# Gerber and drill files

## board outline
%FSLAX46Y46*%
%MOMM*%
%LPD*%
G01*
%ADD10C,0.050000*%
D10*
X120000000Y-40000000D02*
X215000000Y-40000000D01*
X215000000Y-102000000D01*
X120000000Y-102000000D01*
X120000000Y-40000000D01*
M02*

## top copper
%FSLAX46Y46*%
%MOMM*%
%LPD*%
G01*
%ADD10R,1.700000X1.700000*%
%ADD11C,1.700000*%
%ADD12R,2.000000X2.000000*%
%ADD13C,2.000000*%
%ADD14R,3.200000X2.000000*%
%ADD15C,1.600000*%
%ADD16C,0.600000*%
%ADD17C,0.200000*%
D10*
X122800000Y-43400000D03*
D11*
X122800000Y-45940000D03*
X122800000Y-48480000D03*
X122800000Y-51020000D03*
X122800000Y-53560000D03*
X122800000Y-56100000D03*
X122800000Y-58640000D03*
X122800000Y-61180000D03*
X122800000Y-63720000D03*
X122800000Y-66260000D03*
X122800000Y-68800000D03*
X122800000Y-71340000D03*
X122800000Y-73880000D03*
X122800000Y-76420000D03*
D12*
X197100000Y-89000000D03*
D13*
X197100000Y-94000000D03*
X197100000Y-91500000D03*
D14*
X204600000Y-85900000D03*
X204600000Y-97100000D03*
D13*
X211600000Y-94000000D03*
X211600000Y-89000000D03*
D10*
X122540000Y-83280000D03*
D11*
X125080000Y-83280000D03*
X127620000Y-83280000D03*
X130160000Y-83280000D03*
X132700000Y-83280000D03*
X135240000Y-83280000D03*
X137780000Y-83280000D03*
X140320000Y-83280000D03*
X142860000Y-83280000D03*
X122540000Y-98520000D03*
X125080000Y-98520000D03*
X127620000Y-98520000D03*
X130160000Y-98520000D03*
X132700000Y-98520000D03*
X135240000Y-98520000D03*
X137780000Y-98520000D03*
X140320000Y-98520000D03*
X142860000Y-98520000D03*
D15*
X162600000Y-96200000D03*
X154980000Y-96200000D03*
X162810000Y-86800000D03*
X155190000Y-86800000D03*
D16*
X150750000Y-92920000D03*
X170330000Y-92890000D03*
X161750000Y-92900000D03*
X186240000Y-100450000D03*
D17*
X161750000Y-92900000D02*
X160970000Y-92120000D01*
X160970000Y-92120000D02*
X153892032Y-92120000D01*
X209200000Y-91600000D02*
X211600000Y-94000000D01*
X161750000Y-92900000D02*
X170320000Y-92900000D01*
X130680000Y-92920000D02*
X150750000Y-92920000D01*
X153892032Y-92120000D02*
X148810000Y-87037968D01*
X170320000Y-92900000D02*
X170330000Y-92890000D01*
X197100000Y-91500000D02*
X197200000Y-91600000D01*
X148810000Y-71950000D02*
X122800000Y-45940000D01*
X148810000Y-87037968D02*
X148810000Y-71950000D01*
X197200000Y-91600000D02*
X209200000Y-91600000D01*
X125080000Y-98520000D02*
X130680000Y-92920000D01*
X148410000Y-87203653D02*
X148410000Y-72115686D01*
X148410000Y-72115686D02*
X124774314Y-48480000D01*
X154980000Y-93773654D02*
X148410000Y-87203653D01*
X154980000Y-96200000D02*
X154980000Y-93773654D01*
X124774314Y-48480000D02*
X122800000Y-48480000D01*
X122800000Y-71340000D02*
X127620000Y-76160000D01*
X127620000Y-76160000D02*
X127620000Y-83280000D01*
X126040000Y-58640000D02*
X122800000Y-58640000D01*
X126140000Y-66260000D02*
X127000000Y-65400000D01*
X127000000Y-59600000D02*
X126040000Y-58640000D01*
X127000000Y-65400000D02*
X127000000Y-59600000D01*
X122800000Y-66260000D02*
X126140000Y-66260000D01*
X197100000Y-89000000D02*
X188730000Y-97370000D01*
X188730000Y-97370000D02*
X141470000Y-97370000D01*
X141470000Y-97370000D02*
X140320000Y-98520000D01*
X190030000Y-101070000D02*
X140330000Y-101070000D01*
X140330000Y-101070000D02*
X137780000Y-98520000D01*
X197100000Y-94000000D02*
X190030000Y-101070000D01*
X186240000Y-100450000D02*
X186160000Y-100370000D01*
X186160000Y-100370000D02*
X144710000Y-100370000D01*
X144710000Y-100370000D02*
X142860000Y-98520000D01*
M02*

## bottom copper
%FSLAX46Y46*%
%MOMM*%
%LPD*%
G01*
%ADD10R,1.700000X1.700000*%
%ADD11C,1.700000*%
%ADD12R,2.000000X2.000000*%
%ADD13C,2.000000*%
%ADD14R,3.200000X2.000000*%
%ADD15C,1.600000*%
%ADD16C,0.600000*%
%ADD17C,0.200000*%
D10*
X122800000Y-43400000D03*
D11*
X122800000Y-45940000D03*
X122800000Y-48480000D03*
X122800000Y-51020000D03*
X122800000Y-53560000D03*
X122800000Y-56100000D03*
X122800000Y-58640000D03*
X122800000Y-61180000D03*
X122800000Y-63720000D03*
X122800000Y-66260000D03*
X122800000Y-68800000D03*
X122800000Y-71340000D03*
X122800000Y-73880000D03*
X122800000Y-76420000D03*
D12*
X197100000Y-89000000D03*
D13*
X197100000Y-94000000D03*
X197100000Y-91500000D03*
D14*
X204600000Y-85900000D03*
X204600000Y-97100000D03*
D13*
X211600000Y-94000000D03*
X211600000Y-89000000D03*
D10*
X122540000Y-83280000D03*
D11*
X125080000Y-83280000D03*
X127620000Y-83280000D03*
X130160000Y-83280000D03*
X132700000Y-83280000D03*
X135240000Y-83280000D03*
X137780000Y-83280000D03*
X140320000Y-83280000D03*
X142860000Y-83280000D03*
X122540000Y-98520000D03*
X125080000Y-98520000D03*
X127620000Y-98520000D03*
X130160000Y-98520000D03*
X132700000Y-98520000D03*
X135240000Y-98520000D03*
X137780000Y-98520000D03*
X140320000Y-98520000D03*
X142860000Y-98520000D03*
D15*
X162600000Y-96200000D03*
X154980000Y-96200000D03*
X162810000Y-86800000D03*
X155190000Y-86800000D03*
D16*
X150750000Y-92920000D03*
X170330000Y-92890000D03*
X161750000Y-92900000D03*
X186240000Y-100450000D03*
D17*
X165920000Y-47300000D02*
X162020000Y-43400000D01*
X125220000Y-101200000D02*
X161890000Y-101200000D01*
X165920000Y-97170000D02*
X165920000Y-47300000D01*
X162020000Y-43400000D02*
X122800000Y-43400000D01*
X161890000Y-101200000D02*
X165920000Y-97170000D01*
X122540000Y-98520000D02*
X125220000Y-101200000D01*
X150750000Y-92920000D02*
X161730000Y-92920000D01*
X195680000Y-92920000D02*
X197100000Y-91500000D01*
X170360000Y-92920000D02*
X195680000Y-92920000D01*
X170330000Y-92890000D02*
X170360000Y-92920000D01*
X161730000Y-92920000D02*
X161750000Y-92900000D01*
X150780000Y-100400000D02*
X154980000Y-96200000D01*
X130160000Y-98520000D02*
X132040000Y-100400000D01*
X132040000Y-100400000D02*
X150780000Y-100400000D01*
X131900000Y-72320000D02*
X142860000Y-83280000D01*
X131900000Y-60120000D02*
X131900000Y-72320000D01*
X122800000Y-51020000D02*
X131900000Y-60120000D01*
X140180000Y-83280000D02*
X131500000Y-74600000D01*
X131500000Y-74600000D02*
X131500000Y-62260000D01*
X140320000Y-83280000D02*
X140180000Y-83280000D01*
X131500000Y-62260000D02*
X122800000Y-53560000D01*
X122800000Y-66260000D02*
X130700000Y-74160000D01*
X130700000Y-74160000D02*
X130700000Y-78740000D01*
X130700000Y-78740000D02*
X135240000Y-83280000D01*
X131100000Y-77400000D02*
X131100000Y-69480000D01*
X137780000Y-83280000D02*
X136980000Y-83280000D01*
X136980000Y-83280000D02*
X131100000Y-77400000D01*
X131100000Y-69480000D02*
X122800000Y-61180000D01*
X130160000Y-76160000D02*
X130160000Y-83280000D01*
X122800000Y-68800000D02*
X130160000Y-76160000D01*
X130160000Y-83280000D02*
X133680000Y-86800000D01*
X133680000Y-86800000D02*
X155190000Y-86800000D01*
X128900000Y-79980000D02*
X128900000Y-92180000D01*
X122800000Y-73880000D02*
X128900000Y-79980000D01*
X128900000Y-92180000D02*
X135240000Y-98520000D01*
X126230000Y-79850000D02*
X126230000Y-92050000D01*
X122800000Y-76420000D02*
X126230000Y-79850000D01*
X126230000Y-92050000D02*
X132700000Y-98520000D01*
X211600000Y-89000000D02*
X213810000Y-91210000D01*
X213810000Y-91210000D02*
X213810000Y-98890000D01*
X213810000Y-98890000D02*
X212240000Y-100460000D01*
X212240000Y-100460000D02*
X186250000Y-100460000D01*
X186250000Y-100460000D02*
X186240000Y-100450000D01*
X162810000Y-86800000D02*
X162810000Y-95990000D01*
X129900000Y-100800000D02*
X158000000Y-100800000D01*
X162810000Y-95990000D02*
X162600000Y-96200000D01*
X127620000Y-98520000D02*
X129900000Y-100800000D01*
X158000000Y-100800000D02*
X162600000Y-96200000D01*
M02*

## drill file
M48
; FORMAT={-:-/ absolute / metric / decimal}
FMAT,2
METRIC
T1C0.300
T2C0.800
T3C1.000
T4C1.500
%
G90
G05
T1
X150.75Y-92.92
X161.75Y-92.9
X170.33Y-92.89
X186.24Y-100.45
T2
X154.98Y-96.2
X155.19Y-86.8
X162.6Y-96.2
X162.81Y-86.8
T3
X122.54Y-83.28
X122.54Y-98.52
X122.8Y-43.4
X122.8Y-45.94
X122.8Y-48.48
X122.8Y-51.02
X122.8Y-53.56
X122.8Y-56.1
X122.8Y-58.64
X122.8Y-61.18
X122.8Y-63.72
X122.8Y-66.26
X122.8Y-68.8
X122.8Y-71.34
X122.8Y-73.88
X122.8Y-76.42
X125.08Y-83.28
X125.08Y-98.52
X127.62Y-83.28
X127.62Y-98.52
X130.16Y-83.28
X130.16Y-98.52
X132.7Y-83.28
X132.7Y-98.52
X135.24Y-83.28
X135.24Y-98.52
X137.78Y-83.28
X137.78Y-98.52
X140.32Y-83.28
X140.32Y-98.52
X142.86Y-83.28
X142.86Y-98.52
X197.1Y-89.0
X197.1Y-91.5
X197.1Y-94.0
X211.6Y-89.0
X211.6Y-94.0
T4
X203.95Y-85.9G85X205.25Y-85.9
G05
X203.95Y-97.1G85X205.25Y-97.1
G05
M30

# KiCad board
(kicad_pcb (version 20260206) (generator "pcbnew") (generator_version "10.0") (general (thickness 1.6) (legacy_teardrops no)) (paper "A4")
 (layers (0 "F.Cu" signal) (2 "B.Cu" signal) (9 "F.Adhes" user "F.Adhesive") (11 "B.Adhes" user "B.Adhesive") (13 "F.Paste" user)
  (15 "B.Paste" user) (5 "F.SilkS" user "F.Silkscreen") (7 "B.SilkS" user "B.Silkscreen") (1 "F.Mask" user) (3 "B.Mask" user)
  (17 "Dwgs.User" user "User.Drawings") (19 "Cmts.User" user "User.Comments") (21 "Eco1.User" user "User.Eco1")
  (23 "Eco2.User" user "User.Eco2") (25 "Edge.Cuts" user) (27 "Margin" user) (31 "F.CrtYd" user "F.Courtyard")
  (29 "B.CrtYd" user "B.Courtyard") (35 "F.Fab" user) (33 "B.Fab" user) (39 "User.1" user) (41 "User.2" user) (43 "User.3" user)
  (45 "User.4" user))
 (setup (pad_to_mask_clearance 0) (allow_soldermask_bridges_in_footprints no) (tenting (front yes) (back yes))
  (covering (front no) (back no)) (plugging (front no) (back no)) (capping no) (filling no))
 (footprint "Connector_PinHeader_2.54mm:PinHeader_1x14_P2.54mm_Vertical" (layer "F.Cu") (at 122.8 43.4)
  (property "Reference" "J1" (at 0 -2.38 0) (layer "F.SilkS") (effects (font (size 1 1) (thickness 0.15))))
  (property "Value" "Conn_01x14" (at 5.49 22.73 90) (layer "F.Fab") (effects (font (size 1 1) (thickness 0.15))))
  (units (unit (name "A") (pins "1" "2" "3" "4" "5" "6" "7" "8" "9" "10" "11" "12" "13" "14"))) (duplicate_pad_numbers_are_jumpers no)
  (pad "1" thru_hole rect (at 0 0) (size 1.7 1.7) (drill 1) (layers "*.Cu" "*.Mask") (remove_unused_layers no) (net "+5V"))
  (pad "2" thru_hole circle (at 0 2.54) (size 1.7 1.7) (drill 1) (layers "*.Cu" "*.Mask") (remove_unused_layers no) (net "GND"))
  (pad "3" thru_hole circle (at 0 5.08) (size 1.7 1.7) (drill 1) (layers "*.Cu" "*.Mask") (remove_unused_layers no) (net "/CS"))
  (pad "4" thru_hole circle (at 0 7.62) (size 1.7 1.7) (drill 1) (layers "*.Cu" "*.Mask") (remove_unused_layers no) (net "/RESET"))
  (pad "5" thru_hole circle (at 0 10.16) (size 1.7 1.7) (drill 1) (layers "*.Cu" "*.Mask") (remove_unused_layers no) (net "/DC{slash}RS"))
  (pad "6" thru_hole circle (at 0 12.7) (size 1.7 1.7) (drill 1) (layers "*.Cu" "*.Mask") (remove_unused_layers no) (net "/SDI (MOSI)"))
  (pad "7" thru_hole circle (at 0 15.24) (size 1.7 1.7) (drill 1) (layers "*.Cu" "*.Mask") (remove_unused_layers no) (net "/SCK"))
  (pad "8" thru_hole circle (at 0 17.78) (size 1.7 1.7) (drill 1) (layers "*.Cu" "*.Mask") (remove_unused_layers no) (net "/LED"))
  (pad "9" thru_hole circle (at 0 20.32) (size 1.7 1.7) (drill 1) (layers "*.Cu" "*.Mask") (remove_unused_layers no)
   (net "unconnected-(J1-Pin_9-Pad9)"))
  (pad "10" thru_hole circle (at 0 22.86) (size 1.7 1.7) (drill 1) (layers "*.Cu" "*.Mask") (remove_unused_layers no) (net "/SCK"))
  (pad "11" thru_hole circle (at 0 25.4) (size 1.7 1.7) (drill 1) (layers "*.Cu" "*.Mask") (remove_unused_layers no) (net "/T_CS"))
  (pad "12" thru_hole circle (at 0 27.94) (size 1.7 1.7) (drill 1) (layers "*.Cu" "*.Mask") (remove_unused_layers no) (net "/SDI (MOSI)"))
  (pad "13" thru_hole circle (at 0 30.48) (size 1.7 1.7) (drill 1) (layers "*.Cu" "*.Mask") (remove_unused_layers no) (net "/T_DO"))
  (pad "14" thru_hole circle (at 0 33.02) (size 1.7 1.7) (drill 1) (layers "*.Cu" "*.Mask") (remove_unused_layers no) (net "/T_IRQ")))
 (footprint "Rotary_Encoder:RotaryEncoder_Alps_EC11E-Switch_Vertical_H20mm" (layer "F.Cu") (at 197.1 89)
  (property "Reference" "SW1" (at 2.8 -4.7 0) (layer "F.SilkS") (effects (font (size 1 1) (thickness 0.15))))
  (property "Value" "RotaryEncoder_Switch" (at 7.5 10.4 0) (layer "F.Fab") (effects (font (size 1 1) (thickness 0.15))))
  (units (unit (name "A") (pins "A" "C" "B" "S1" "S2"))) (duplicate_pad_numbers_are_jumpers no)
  (pad "A" thru_hole rect (at 0 0) (size 2 2) (drill 1) (layers "*.Cu" "*.Mask") (remove_unused_layers no) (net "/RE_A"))
  (pad "B" thru_hole circle (at 0 5) (size 2 2) (drill 1) (layers "*.Cu" "*.Mask") (remove_unused_layers no) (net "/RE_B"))
  (pad "C" thru_hole circle (at 0 2.5) (size 2 2) (drill 1) (layers "*.Cu" "*.Mask") (remove_unused_layers no) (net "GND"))
  (pad "MP" thru_hole rect (at 7.5 -3.1) (size 3.2 2) (drill oval 2.8 1.5) (layers "*.Cu" "*.Mask") (remove_unused_layers no))
  (pad "MP" thru_hole rect (at 7.5 8.1) (size 3.2 2) (drill oval 2.8 1.5) (layers "*.Cu" "*.Mask") (remove_unused_layers no))
  (pad "S1" thru_hole circle (at 14.5 5) (size 2 2) (drill 1) (layers "*.Cu" "*.Mask") (remove_unused_layers no) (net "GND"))
  (pad "S2" thru_hole circle (at 14.5 0) (size 2 2) (drill 1) (layers "*.Cu" "*.Mask") (remove_unused_layers no) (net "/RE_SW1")))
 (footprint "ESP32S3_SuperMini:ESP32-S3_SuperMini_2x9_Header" (layer "B.Cu") (at 132.7 90.9 -90)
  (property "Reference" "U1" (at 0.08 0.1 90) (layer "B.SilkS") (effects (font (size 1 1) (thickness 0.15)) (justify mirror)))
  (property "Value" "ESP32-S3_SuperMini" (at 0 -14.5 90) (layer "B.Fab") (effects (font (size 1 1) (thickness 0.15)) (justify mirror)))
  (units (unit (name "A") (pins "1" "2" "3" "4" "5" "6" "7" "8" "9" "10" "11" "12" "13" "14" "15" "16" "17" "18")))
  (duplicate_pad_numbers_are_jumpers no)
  (pad "1" thru_hole rect (at -7.62 10.16 270) (size 1.7 1.7) (drill 1) (layers "*.Cu" "*.Mask") (remove_unused_layers no)
   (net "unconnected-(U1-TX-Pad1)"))
  (pad "2" thru_hole circle (at -7.62 7.62 270) (size 1.7 1.7) (drill 1) (layers "*.Cu" "*.Mask") (remove_unused_layers no)
   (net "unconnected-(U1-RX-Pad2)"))
  (pad "3" thru_hole circle (at -7.62 5.08 270) (size 1.7 1.7) (drill 1) (layers "*.Cu" "*.Mask") (remove_unused_layers no)
   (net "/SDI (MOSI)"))
  (pad "4" thru_hole circle (at -7.62 2.54 270) (size 1.7 1.7) (drill 1) (layers "*.Cu" "*.Mask") (remove_unused_layers no) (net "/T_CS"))
  (pad "5" thru_hole circle (at -7.62 0 270) (size 1.7 1.7) (drill 1) (layers "*.Cu" "*.Mask") (remove_unused_layers no)
   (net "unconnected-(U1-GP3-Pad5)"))
  (pad "6" thru_hole circle (at -7.62 -2.54 270) (size 1.7 1.7) (drill 1) (layers "*.Cu" "*.Mask") (remove_unused_layers no) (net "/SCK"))
  (pad "7" thru_hole circle (at -7.62 -5.08 270) (size 1.7 1.7) (drill 1) (layers "*.Cu" "*.Mask") (remove_unused_layers no) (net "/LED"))
  (pad "8" thru_hole circle (at -7.62 -7.62 270) (size 1.7 1.7) (drill 1) (layers "*.Cu" "*.Mask") (remove_unused_layers no)
   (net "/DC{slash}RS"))
  (pad "9" thru_hole circle (at -7.62 -10.16 270) (size 1.7 1.7) (drill 1) (layers "*.Cu" "*.Mask") (remove_unused_layers no) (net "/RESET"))
  (pad "10" thru_hole circle (at 7.62 10.16 270) (size 1.7 1.7) (drill 1) (layers "*.Cu" "*.Mask") (remove_unused_layers no) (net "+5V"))
  (pad "11" thru_hole circle (at 7.62 7.62 270) (size 1.7 1.7) (drill 1) (layers "*.Cu" "*.Mask") (remove_unused_layers no) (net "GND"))
  (pad "12" thru_hole circle (at 7.62 5.08 270) (size 1.7 1.7) (drill 1) (layers "*.Cu" "*.Mask") (remove_unused_layers no) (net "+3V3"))
  (pad "13" thru_hole circle (at 7.62 2.54 270) (size 1.7 1.7) (drill 1) (layers "*.Cu" "*.Mask") (remove_unused_layers no) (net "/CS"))
  (pad "14" thru_hole circle (at 7.62 0 270) (size 1.7 1.7) (drill 1) (layers "*.Cu" "*.Mask") (remove_unused_layers no) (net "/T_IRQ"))
  (pad "15" thru_hole circle (at 7.62 -2.54 270) (size 1.7 1.7) (drill 1) (layers "*.Cu" "*.Mask") (remove_unused_layers no) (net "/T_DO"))
  (pad "16" thru_hole circle (at 7.62 -5.08 270) (size 1.7 1.7) (drill 1) (layers "*.Cu" "*.Mask") (remove_unused_layers no) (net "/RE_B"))
  (pad "17" thru_hole circle (at 7.62 -7.62 270) (size 1.7 1.7) (drill 1) (layers "*.Cu" "*.Mask") (remove_unused_layers no) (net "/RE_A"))
  (pad "18" thru_hole circle (at 7.62 -10.16 270) (size 1.7 1.7) (drill 1) (layers "*.Cu" "*.Mask") (remove_unused_layers no)
   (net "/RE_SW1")))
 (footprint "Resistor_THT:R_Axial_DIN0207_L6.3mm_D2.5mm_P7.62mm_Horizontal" (layer "B.Cu") (at 162.6 96.2 180)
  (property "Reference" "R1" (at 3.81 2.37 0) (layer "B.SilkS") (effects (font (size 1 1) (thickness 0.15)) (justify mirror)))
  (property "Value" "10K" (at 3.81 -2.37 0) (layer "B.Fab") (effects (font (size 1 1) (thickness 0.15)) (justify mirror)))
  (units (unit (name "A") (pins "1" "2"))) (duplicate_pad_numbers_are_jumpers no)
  (pad "1" thru_hole circle (at 0 0 180) (size 1.6 1.6) (drill 0.8) (layers "*.Cu" "*.Mask") (remove_unused_layers no) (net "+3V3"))
  (pad "2" thru_hole circle (at 7.62 0 180) (size 1.6 1.6) (drill 0.8) (layers "*.Cu" "*.Mask") (remove_unused_layers no) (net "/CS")))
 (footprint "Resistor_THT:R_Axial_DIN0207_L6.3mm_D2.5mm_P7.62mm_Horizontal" (layer "B.Cu") (at 162.81 86.8 180)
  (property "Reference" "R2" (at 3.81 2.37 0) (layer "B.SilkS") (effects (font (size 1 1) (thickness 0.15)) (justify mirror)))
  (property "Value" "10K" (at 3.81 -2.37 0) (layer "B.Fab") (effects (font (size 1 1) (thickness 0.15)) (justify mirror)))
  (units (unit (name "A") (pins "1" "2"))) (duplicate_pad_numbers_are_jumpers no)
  (pad "1" thru_hole circle (at 0 0 180) (size 1.6 1.6) (drill 0.8) (layers "*.Cu" "*.Mask") (remove_unused_layers no) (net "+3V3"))
  (pad "2" thru_hole circle (at 7.62 0 180) (size 1.6 1.6) (drill 0.8) (layers "*.Cu" "*.Mask") (remove_unused_layers no) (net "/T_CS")))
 (gr_rect (start 120 40) (end 215 102) (stroke (width 0.05) (type solid)) (fill no) (layer "Edge.Cuts"))
 (segment (start 165.92 47.3) (end 162.02 43.4) (width 0.2) (layer "B.Cu") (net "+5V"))
 (segment (start 125.22 101.2) (end 161.89 101.2) (width 0.2) (layer "B.Cu") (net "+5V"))
 (segment (start 165.92 97.17) (end 165.92 47.3) (width 0.2) (layer "B.Cu") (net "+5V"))
 (segment (start 162.02 43.4) (end 122.8 43.4) (width 0.2) (layer "B.Cu") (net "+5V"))
 (segment (start 161.89 101.2) (end 165.92 97.17) (width 0.2) (layer "B.Cu") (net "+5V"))
 (segment (start 122.54 98.52) (end 125.22 101.2) (width 0.2) (layer "B.Cu") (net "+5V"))
 (segment (start 161.75 92.9) (end 160.97 92.12) (width 0.2) (layer "F.Cu") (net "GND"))
 (segment (start 160.97 92.12) (end 153.892032 92.12) (width 0.2) (layer "F.Cu") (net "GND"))
 (segment (start 209.2 91.6) (end 211.6 94) (width 0.2) (layer "F.Cu") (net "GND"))
 (segment (start 161.75 92.9) (end 170.32 92.9) (width 0.2) (layer "F.Cu") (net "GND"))
 (segment (start 130.68 92.92) (end 150.75 92.92) (width 0.2) (layer "F.Cu") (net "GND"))
 (segment (start 153.892032 92.12) (end 148.81 87.037968) (width 0.2) (layer "F.Cu") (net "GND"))
 (segment (start 170.32 92.9) (end 170.33 92.89) (width 0.2) (layer "F.Cu") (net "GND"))
 (segment (start 197.1 91.5) (end 197.2 91.6) (width 0.2) (layer "F.Cu") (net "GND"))
 (segment (start 148.81 71.95) (end 122.8 45.94) (width 0.2) (layer "F.Cu") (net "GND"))
 (segment (start 148.81 87.037968) (end 148.81 71.95) (width 0.2) (layer "F.Cu") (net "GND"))
 (segment (start 197.2 91.6) (end 209.2 91.6) (width 0.2) (layer "F.Cu") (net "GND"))
 (segment (start 125.08 98.52) (end 130.68 92.92) (width 0.2) (layer "F.Cu") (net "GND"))
 (via (at 150.75 92.92) (size 0.6) (drill 0.3) (layers "F.Cu" "B.Cu") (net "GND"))
 (via (at 170.33 92.89) (size 0.6) (drill 0.3) (layers "F.Cu" "B.Cu") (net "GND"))
 (via (at 161.75 92.9) (size 0.6) (drill 0.3) (layers "F.Cu" "B.Cu") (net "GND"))
 (segment (start 150.75 92.92) (end 161.73 92.92) (width 0.2) (layer "B.Cu") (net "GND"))
 (segment (start 195.68 92.92) (end 197.1 91.5) (width 0.2) (layer "B.Cu") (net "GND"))
 (segment (start 170.36 92.92) (end 195.68 92.92) (width 0.2) (layer "B.Cu") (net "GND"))
 (segment (start 170.33 92.89) (end 170.36 92.92) (width 0.2) (layer "B.Cu") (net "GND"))
 (segment (start 161.73 92.92) (end 161.75 92.9) (width 0.2) (layer "B.Cu") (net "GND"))
 (segment (start 148.41 87.203653) (end 148.41 72.115686) (width 0.2) (layer "F.Cu") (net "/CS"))
 (segment (start 148.41 72.115686) (end 124.774314 48.48) (width 0.2) (layer "F.Cu") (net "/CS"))
 (segment (start 154.98 93.773654) (end 148.41 87.203653) (width 0.2) (layer "F.Cu") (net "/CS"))
 (segment (start 154.98 96.2) (end 154.98 93.773654) (width 0.2) (layer "F.Cu") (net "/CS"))
 (segment (start 124.774314 48.48) (end 122.8 48.48) (width 0.2) (layer "F.Cu") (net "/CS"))
 (segment (start 150.78 100.4) (end 154.98 96.2) (width 0.2) (layer "B.Cu") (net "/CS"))
 (segment (start 130.16 98.52) (end 132.04 100.4) (width 0.2) (layer "B.Cu") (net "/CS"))
 (segment (start 132.04 100.4) (end 150.78 100.4) (width 0.2) (layer "B.Cu") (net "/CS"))
 (segment (start 131.9 72.32) (end 142.86 83.28) (width 0.2) (layer "B.Cu") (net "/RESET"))
 (segment (start 131.9 60.12) (end 131.9 72.32) (width 0.2) (layer "B.Cu") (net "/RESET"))
 (segment (start 122.8 51.02) (end 131.9 60.12) (width 0.2) (layer "B.Cu") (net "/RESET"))
 (segment (start 140.18 83.28) (end 131.5 74.6) (width 0.2) (layer "B.Cu") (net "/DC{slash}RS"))
 (segment (start 131.5 74.6) (end 131.5 62.26) (width 0.2) (layer "B.Cu") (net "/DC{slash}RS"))
 (segment (start 140.32 83.28) (end 140.18 83.28) (width 0.2) (layer "B.Cu") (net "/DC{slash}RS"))
 (segment (start 131.5 62.26) (end 122.8 53.56) (width 0.2) (layer "B.Cu") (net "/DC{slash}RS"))
 (segment (start 122.8 71.34) (end 127.62 76.16) (width 0.2) (layer "F.Cu") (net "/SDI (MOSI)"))
 (segment (start 127.62 76.16) (end 127.62 83.28) (width 0.2) (layer "F.Cu") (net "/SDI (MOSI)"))
 (segment (start 126.04 58.64) (end 122.8 58.64) (width 0.2) (layer "F.Cu") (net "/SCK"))
 (segment (start 126.14 66.26) (end 127 65.4) (width 0.2) (layer "F.Cu") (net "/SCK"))
 (segment (start 127 59.6) (end 126.04 58.64) (width 0.2) (layer "F.Cu") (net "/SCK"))
 (segment (start 127 65.4) (end 127 59.6) (width 0.2) (layer "F.Cu") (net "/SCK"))
 (segment (start 122.8 66.26) (end 126.14 66.26) (width 0.2) (layer "F.Cu") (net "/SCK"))
 (segment (start 122.8 66.26) (end 130.7 74.16) (width 0.2) (layer "B.Cu") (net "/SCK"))
 (segment (start 130.7 74.16) (end 130.7 78.74) (width 0.2) (layer "B.Cu") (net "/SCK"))
 (segment (start 130.7 78.74) (end 135.24 83.28) (width 0.2) (layer "B.Cu") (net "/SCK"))
 (segment (start 131.1 77.4) (end 131.1 69.48) (width 0.2) (layer "B.Cu") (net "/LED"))
 (segment (start 137.78 83.28) (end 136.98 83.28) (width 0.2) (layer "B.Cu") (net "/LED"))
 (segment (start 136.98 83.28) (end 131.1 77.4) (width 0.2) (layer "B.Cu") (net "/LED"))
 (segment (start 131.1 69.48) (end 122.8 61.18) (width 0.2) (layer "B.Cu") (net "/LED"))
 (segment (start 130.16 76.16) (end 130.16 83.28) (width 0.2) (layer "B.Cu") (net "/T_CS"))
 (segment (start 122.8 68.8) (end 130.16 76.16) (width 0.2) (layer "B.Cu") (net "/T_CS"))
 (segment (start 130.16 83.28) (end 133.68 86.8) (width 0.2) (layer "B.Cu") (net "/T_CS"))
 (segment (start 133.68 86.8) (end 155.19 86.8) (width 0.2) (layer "B.Cu") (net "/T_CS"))
 (segment (start 128.9 79.98) (end 128.9 92.18) (width 0.2) (layer "B.Cu") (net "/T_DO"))
 (segment (start 122.8 73.88) (end 128.9 79.98) (width 0.2) (layer "B.Cu") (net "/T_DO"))
 (segment (start 128.9 92.18) (end 135.24 98.52) (width 0.2) (layer "B.Cu") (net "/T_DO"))
 (segment (start 126.23 79.85) (end 126.23 92.05) (width 0.2) (layer "B.Cu") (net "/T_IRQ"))
 (segment (start 122.8 76.42) (end 126.23 79.85) (width 0.2) (layer "B.Cu") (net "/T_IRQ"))
 (segment (start 126.23 92.05) (end 132.7 98.52) (width 0.2) (layer "B.Cu") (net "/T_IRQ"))
 (segment (start 197.1 89) (end 188.73 97.37) (width 0.2) (layer "F.Cu") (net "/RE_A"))
 (segment (start 188.73 97.37) (end 141.47 97.37) (width 0.2) (layer "F.Cu") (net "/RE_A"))
 (segment (start 141.47 97.37) (end 140.32 98.52) (width 0.2) (layer "F.Cu") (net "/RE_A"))
 (segment (start 190.03 101.07) (end 140.33 101.07) (width 0.2) (layer "F.Cu") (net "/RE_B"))
 (segment (start 140.33 101.07) (end 137.78 98.52) (width 0.2) (layer "F.Cu") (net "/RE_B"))
 (segment (start 197.1 94) (end 190.03 101.07) (width 0.2) (layer "F.Cu") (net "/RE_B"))
 (segment (start 186.24 100.45) (end 186.16 100.37) (width 0.2) (layer "F.Cu") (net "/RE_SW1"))
 (segment (start 186.16 100.37) (end 144.71 100.37) (width 0.2) (layer "F.Cu") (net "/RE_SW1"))
 (segment (start 144.71 100.37) (end 142.86 98.52) (width 0.2) (layer "F.Cu") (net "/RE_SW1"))
 (via (at 186.24 100.45) (size 0.6) (drill 0.3) (layers "F.Cu" "B.Cu") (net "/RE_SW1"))
 (segment (start 211.6 89) (end 213.81 91.21) (width 0.2) (layer "B.Cu") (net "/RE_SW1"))
 (segment (start 213.81 91.21) (end 213.81 98.89) (width 0.2) (layer "B.Cu") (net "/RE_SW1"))
 (segment (start 213.81 98.89) (end 212.24 100.46) (width 0.2) (layer "B.Cu") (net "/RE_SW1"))
 (segment (start 212.24 100.46) (end 186.25 100.46) (width 0.2) (layer "B.Cu") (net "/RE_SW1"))
 (segment (start 186.25 100.46) (end 186.24 100.45) (width 0.2) (layer "B.Cu") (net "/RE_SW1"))
 (segment (start 162.81 86.8) (end 162.81 95.99) (width 0.2) (layer "B.Cu") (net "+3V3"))
 (segment (start 129.9 100.8) (end 158 100.8) (width 0.2) (layer "B.Cu") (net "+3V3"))
 (segment (start 162.81 95.99) (end 162.6 96.2) (width 0.2) (layer "B.Cu") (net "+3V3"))
 (segment (start 127.62 98.52) (end 129.9 100.8) (width 0.2) (layer "B.Cu") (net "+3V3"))
 (segment (start 158 100.8) (end 162.6 96.2) (width 0.2) (layer "B.Cu") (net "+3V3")))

